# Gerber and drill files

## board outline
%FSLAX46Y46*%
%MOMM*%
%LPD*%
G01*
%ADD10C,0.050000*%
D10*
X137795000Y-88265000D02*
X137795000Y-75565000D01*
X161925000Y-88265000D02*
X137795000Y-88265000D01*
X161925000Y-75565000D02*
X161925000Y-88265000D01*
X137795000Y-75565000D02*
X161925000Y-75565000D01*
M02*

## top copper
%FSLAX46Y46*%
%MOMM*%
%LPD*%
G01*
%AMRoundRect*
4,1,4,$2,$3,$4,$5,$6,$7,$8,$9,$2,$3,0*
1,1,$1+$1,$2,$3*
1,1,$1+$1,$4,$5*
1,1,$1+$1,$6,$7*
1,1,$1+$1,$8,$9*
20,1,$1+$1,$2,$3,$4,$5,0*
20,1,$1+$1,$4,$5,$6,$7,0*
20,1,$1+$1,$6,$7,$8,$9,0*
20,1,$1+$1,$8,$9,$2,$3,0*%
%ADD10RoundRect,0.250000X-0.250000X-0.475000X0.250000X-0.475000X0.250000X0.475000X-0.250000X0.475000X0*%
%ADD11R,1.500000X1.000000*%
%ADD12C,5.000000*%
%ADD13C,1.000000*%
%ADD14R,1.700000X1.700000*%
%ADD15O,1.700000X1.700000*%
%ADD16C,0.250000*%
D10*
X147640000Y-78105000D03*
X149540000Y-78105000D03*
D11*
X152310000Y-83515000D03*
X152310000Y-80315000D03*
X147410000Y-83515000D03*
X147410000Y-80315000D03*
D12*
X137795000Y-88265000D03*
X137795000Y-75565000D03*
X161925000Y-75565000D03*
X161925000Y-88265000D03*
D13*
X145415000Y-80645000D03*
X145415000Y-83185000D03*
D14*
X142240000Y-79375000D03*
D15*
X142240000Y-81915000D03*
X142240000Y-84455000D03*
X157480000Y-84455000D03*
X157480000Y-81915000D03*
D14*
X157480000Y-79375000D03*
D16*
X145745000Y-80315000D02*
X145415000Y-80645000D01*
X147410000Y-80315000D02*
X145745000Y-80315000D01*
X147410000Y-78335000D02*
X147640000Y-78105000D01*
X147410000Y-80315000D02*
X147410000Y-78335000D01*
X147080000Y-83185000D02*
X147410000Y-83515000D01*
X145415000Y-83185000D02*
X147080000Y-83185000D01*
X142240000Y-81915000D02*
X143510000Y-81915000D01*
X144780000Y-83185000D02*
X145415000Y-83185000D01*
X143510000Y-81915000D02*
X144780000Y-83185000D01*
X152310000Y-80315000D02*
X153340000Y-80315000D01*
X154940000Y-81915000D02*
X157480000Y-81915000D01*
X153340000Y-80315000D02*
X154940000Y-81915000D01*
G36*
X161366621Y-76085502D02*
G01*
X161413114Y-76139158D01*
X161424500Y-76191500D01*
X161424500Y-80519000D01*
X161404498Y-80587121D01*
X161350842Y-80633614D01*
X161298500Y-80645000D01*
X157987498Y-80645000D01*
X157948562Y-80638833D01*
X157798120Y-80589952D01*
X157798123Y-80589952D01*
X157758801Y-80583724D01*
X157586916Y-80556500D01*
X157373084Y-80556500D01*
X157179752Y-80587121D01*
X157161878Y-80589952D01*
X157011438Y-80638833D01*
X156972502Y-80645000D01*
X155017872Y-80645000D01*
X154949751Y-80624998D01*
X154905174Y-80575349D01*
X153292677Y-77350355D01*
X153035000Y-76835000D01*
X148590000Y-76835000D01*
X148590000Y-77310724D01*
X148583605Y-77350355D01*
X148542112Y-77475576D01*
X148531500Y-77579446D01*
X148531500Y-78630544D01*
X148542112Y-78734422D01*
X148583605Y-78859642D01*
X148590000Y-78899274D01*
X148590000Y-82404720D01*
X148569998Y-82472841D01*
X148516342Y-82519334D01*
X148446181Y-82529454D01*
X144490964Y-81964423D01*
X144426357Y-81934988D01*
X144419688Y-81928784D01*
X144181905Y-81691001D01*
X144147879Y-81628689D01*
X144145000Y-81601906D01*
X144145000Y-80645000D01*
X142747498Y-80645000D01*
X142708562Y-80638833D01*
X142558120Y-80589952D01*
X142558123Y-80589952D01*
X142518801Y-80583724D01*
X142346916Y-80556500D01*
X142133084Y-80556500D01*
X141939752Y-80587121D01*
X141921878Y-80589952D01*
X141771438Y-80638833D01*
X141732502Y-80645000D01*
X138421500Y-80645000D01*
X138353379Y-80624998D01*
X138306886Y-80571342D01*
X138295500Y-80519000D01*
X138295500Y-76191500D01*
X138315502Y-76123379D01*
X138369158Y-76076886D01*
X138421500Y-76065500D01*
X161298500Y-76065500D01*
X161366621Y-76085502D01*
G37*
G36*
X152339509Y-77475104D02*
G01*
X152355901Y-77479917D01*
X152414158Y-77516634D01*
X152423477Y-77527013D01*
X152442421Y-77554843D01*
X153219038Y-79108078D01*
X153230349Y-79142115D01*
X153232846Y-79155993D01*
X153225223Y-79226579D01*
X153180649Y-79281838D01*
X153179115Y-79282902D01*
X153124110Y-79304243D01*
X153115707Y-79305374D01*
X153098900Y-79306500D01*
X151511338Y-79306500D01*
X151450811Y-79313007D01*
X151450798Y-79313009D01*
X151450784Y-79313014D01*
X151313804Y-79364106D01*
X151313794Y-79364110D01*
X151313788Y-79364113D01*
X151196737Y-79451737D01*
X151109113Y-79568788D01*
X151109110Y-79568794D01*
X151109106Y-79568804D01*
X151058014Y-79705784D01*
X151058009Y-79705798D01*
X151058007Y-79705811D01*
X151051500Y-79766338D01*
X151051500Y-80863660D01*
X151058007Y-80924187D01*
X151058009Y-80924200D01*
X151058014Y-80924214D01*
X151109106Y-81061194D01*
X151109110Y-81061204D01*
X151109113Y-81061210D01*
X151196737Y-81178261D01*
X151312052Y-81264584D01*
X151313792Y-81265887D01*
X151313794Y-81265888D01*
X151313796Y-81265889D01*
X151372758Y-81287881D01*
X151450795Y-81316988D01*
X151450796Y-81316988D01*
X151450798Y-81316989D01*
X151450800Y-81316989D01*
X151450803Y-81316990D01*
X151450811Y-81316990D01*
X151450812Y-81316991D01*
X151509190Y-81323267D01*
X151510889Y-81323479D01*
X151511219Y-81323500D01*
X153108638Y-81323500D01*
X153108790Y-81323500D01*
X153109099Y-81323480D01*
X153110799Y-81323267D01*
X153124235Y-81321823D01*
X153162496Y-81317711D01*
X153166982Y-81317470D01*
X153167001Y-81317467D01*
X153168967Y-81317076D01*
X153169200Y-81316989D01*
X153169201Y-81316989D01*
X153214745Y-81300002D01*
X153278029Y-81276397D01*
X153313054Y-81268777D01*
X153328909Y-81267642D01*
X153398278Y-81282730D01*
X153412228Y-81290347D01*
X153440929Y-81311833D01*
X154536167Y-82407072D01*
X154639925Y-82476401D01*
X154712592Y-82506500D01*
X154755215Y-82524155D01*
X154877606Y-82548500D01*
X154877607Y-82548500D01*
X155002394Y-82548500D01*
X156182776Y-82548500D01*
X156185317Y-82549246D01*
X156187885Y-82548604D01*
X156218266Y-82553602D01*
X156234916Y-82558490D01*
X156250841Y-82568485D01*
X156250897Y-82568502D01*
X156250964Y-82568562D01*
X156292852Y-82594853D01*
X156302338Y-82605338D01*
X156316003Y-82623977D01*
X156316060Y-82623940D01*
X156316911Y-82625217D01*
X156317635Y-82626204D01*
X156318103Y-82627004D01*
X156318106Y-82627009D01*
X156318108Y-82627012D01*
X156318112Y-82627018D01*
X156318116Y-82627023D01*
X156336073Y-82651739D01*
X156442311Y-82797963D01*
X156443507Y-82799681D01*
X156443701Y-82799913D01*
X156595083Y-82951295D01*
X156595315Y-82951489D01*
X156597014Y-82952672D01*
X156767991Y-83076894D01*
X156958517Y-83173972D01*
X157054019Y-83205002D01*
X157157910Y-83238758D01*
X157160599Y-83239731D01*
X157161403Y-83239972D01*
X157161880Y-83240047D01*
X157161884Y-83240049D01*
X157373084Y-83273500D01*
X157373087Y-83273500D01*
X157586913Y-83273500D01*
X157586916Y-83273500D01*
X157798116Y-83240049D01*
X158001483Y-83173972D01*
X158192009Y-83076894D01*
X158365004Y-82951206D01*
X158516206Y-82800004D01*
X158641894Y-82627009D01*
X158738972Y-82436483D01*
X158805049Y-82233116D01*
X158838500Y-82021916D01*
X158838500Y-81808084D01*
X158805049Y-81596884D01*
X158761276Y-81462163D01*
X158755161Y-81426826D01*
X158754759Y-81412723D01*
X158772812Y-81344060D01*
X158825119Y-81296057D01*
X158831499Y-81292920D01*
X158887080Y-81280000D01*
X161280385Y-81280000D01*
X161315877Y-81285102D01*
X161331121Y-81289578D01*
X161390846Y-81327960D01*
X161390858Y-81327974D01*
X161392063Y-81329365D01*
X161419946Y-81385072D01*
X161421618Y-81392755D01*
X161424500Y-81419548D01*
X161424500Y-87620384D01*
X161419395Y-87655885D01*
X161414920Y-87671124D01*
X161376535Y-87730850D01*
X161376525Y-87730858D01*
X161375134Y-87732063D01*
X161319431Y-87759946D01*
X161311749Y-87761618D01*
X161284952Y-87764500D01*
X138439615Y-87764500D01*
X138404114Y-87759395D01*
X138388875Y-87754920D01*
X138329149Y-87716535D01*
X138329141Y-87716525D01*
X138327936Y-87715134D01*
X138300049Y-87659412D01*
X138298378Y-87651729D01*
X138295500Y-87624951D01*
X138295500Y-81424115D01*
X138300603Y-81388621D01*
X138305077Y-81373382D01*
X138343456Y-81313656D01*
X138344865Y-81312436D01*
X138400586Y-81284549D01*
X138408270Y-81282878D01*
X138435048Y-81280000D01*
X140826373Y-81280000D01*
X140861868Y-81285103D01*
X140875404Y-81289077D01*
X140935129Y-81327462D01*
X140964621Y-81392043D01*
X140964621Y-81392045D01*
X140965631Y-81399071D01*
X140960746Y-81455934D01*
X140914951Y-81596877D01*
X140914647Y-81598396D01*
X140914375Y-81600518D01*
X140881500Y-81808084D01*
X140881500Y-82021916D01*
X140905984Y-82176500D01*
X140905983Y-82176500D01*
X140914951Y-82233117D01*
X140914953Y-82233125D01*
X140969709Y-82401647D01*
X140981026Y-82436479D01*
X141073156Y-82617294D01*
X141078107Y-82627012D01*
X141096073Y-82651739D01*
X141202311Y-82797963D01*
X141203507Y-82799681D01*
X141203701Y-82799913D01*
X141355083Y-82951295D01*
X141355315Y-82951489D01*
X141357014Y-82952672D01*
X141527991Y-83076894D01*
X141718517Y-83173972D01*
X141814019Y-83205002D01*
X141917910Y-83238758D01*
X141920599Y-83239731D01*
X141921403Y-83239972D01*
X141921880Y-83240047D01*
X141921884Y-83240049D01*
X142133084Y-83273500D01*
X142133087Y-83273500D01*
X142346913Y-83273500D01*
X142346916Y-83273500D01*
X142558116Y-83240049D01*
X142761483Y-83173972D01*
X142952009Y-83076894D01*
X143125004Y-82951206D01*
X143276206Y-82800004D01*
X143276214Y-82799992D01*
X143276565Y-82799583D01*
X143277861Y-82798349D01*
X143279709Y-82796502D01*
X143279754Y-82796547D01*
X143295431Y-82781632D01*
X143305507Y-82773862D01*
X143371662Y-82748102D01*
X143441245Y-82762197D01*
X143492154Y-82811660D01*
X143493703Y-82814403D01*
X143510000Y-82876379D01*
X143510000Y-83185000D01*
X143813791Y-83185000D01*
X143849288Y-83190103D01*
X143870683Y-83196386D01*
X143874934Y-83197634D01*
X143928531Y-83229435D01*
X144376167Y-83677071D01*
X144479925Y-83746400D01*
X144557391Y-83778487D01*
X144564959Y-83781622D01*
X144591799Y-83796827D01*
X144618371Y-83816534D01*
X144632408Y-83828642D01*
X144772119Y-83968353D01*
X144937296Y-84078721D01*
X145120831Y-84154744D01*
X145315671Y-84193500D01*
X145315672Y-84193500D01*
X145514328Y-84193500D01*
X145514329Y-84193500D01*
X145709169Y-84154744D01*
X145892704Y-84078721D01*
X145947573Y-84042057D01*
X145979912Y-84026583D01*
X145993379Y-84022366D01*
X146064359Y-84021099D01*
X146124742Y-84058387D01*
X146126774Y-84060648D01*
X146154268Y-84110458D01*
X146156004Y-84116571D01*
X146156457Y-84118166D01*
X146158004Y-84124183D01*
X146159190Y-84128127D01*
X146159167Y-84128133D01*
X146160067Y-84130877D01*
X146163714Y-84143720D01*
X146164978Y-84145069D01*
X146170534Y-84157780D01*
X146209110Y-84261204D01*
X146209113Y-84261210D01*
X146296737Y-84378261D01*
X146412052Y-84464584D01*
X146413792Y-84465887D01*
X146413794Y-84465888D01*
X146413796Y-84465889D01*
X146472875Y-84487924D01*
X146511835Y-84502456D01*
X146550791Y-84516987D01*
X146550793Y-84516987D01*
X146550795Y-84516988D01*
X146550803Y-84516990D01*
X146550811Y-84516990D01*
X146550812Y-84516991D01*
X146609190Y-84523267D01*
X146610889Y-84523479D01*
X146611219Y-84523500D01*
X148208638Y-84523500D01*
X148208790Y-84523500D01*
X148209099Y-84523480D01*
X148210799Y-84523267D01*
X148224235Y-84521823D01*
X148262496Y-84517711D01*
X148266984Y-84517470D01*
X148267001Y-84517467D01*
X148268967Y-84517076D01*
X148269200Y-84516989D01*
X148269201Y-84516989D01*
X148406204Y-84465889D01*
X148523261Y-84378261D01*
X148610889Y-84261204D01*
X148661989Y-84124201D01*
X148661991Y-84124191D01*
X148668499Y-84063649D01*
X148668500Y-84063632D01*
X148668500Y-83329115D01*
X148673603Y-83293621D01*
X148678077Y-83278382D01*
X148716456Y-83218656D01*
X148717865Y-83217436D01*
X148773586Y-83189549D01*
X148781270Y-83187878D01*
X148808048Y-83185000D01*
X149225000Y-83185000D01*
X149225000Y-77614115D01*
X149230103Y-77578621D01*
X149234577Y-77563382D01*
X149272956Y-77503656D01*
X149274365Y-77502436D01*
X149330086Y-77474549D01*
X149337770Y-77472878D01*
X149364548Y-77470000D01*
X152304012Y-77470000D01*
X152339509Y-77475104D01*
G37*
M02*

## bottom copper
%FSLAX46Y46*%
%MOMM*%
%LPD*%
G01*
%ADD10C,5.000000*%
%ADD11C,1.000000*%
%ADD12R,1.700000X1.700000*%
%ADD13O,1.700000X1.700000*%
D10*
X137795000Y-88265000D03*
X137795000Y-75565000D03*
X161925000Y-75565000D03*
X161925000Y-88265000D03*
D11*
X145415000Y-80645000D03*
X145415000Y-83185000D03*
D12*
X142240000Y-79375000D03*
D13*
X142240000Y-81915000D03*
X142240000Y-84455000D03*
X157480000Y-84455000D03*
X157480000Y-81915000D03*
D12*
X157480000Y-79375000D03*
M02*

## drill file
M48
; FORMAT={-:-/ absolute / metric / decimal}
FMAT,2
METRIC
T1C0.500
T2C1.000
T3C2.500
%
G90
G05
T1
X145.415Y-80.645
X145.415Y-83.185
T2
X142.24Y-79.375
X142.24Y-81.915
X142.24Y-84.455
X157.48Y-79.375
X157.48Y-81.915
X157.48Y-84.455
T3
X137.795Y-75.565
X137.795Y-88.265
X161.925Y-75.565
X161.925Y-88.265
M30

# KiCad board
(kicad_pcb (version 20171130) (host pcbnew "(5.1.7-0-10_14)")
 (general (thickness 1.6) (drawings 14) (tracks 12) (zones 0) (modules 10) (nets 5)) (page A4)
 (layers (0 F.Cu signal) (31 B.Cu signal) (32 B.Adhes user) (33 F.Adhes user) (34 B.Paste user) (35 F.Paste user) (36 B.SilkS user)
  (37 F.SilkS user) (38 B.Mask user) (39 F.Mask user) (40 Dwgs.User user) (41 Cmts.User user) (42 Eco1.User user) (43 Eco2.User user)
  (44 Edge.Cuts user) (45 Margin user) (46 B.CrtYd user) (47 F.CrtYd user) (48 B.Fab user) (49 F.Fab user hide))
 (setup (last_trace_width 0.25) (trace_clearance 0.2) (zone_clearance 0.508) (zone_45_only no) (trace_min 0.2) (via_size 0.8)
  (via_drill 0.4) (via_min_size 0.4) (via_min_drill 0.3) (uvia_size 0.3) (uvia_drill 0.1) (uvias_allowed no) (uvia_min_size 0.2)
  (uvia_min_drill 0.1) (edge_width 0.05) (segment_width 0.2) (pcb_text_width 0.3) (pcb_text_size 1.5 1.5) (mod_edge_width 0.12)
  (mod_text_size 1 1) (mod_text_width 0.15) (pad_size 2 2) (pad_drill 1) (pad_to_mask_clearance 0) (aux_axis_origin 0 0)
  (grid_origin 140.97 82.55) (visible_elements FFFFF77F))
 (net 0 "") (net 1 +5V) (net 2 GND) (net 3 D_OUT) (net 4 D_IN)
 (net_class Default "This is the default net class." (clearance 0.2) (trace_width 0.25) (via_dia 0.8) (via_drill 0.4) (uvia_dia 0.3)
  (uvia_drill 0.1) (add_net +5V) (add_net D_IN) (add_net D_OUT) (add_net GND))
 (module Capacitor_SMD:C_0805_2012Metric (layer F.Cu) (at 148.59 78.105)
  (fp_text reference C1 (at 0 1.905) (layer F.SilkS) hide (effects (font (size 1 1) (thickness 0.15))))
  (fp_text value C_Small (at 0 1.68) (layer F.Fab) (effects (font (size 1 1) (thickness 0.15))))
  (pad 1 smd roundrect (at -0.95 0) (size 1 1.45) (layers F.Cu F.Paste F.Mask) (roundrect_rratio 0.25) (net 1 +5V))
  (pad 2 smd roundrect (at 0.95 0) (size 1 1.45) (layers F.Cu F.Paste F.Mask) (roundrect_rratio 0.25) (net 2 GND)))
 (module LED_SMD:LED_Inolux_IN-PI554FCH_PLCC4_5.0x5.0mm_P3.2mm (layer F.Cu) (at 149.86 81.915)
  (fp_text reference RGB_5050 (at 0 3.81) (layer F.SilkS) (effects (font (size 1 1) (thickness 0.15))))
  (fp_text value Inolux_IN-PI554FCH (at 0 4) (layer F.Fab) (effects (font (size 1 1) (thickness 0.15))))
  (pad 3 smd rect (at 2.45 1.6) (size 1.5 1) (layers F.Cu F.Paste F.Mask) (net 2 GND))
  (pad 4 smd rect (at 2.45 -1.6) (size 1.5 1) (layers F.Cu F.Paste F.Mask) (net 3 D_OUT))
  (pad 2 smd rect (at -2.45 1.6) (size 1.5 1) (layers F.Cu F.Paste F.Mask) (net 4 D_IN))
  (pad 1 smd rect (at -2.45 -1.6) (size 1.5 1) (layers F.Cu F.Paste F.Mask) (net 1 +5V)))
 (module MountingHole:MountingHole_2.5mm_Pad (layer F.Cu) (at 137.795 88.265)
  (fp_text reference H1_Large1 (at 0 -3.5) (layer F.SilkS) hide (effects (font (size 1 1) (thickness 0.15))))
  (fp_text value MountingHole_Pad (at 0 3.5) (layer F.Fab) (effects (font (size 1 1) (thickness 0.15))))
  (pad 1 thru_hole circle (at 0 0) (size 5 5) (drill 2.5) (layers *.Cu *.Mask) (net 2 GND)))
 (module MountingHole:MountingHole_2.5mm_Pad (layer F.Cu) (at 137.795 75.565)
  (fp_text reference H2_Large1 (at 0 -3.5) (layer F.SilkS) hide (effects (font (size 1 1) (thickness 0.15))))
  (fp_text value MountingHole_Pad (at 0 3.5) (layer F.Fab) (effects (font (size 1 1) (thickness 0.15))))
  (pad 1 thru_hole circle (at 0 0) (size 5 5) (drill 2.5) (layers *.Cu *.Mask) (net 1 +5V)))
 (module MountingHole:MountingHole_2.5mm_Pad (layer F.Cu) (at 161.925 75.565)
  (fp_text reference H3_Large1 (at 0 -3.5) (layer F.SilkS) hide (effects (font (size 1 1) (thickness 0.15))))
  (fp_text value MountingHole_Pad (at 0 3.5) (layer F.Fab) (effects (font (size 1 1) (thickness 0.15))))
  (pad 1 thru_hole circle (at 0 0) (size 5 5) (drill 2.5) (layers *.Cu *.Mask) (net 1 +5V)))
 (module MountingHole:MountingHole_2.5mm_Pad (layer F.Cu) (at 161.925 88.265)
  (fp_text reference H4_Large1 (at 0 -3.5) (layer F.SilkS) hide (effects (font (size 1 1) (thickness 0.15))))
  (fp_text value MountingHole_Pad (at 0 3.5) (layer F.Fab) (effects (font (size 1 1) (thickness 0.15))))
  (pad 1 thru_hole circle (at 0 0) (size 5 5) (drill 2.5) (layers *.Cu *.Mask) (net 2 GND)))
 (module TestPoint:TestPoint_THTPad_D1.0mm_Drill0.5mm (layer F.Cu) (at 145.415 80.645)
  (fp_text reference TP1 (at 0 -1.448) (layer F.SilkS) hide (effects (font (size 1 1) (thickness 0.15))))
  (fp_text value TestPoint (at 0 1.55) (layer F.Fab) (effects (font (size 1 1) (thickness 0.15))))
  (pad 1 thru_hole circle (at 0 0) (size 1 1) (drill 0.5) (layers *.Cu *.Mask) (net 1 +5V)))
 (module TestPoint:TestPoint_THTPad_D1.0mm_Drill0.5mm (layer F.Cu) (at 145.415 83.185)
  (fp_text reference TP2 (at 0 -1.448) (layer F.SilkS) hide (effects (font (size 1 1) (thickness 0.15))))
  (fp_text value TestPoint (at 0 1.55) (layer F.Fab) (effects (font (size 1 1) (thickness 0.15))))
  (pad 1 thru_hole circle (at 0 0) (size 1 1) (drill 0.5) (layers *.Cu *.Mask) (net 4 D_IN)))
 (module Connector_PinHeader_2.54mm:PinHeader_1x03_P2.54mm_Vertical (layer F.Cu) (at 142.24 79.375)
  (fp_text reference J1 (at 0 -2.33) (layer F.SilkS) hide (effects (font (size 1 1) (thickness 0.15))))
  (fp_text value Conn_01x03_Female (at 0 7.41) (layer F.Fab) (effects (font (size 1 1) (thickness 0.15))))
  (pad 1 thru_hole rect (at 0 0) (size 1.7 1.7) (drill 1) (layers *.Cu *.Mask) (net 1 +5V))
  (pad 2 thru_hole oval (at 0 2.54) (size 1.7 1.7) (drill 1) (layers *.Cu *.Mask) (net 4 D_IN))
  (pad 3 thru_hole oval (at 0 5.08) (size 1.7 1.7) (drill 1) (layers *.Cu *.Mask) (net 2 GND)))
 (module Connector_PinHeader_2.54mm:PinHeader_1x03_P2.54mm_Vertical (layer F.Cu) (at 157.48 79.375)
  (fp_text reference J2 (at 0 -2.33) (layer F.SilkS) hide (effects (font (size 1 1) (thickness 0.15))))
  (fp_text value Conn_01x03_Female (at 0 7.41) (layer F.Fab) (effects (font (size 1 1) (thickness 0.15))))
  (pad 3 thru_hole oval (at 0 5.08) (size 1.7 1.7) (drill 1) (layers *.Cu *.Mask) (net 2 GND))
  (pad 2 thru_hole oval (at 0 2.54) (size 1.7 1.7) (drill 1) (layers *.Cu *.Mask) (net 3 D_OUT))
  (pad 1 thru_hole rect (at 0 0) (size 1.7 1.7) (drill 1) (layers *.Cu *.Mask) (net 1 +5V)))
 (gr_line (start 137.795 88.265) (end 137.795 75.565) (layer Edge.Cuts) (width 0.05))
 (gr_line (start 161.925 88.265) (end 137.795 88.265) (layer Edge.Cuts) (width 0.05))
 (gr_line (start 161.925 75.565) (end 161.925 88.265) (layer Edge.Cuts) (width 0.05))
 (gr_line (start 137.795 75.565) (end 161.925 75.565) (layer Edge.Cuts) (width 0.05))
 (segment (start 145.745 80.315) (end 145.415 80.645) (width 0.25) (layer F.Cu) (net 1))
 (segment (start 147.41 80.315) (end 145.745 80.315) (width 0.25) (layer F.Cu) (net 1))
 (segment (start 147.41 78.335) (end 147.64 78.105) (width 0.25) (layer F.Cu) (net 1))
 (segment (start 147.41 80.315) (end 147.41 78.335) (width 0.25) (layer F.Cu) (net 1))
 (segment (start 147.08 83.185) (end 147.41 83.515) (width 0.25) (layer F.Cu) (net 4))
 (segment (start 145.415 83.185) (end 147.08 83.185) (width 0.25) (layer F.Cu) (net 4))
 (segment (start 142.24 81.915) (end 143.51 81.915) (width 0.25) (layer F.Cu) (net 4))
 (segment (start 144.78 83.185) (end 145.415 83.185) (width 0.25) (layer F.Cu) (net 4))
 (segment (start 143.51 81.915) (end 144.78 83.185) (width 0.25) (layer F.Cu) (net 4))
 (segment (start 152.31 80.315) (end 153.34 80.315) (width 0.25) (layer F.Cu) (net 3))
 (segment (start 154.94 81.915) (end 157.48 81.915) (width 0.25) (layer F.Cu) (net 3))
 (segment (start 153.34 80.315) (end 154.94 81.915) (width 0.25) (layer F.Cu) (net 3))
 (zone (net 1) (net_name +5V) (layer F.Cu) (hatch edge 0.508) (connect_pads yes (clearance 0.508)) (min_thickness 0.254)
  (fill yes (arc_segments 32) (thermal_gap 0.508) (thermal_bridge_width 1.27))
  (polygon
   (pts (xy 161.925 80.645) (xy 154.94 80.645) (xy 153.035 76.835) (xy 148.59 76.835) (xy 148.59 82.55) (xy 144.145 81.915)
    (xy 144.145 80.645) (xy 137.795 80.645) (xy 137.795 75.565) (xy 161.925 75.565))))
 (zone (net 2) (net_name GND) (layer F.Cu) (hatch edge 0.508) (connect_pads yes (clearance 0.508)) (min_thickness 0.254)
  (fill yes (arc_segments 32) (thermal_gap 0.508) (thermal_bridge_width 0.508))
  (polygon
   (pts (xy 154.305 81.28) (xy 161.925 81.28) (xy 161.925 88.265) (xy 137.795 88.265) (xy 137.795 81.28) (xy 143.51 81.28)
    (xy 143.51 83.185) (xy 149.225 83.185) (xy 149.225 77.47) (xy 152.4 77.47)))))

